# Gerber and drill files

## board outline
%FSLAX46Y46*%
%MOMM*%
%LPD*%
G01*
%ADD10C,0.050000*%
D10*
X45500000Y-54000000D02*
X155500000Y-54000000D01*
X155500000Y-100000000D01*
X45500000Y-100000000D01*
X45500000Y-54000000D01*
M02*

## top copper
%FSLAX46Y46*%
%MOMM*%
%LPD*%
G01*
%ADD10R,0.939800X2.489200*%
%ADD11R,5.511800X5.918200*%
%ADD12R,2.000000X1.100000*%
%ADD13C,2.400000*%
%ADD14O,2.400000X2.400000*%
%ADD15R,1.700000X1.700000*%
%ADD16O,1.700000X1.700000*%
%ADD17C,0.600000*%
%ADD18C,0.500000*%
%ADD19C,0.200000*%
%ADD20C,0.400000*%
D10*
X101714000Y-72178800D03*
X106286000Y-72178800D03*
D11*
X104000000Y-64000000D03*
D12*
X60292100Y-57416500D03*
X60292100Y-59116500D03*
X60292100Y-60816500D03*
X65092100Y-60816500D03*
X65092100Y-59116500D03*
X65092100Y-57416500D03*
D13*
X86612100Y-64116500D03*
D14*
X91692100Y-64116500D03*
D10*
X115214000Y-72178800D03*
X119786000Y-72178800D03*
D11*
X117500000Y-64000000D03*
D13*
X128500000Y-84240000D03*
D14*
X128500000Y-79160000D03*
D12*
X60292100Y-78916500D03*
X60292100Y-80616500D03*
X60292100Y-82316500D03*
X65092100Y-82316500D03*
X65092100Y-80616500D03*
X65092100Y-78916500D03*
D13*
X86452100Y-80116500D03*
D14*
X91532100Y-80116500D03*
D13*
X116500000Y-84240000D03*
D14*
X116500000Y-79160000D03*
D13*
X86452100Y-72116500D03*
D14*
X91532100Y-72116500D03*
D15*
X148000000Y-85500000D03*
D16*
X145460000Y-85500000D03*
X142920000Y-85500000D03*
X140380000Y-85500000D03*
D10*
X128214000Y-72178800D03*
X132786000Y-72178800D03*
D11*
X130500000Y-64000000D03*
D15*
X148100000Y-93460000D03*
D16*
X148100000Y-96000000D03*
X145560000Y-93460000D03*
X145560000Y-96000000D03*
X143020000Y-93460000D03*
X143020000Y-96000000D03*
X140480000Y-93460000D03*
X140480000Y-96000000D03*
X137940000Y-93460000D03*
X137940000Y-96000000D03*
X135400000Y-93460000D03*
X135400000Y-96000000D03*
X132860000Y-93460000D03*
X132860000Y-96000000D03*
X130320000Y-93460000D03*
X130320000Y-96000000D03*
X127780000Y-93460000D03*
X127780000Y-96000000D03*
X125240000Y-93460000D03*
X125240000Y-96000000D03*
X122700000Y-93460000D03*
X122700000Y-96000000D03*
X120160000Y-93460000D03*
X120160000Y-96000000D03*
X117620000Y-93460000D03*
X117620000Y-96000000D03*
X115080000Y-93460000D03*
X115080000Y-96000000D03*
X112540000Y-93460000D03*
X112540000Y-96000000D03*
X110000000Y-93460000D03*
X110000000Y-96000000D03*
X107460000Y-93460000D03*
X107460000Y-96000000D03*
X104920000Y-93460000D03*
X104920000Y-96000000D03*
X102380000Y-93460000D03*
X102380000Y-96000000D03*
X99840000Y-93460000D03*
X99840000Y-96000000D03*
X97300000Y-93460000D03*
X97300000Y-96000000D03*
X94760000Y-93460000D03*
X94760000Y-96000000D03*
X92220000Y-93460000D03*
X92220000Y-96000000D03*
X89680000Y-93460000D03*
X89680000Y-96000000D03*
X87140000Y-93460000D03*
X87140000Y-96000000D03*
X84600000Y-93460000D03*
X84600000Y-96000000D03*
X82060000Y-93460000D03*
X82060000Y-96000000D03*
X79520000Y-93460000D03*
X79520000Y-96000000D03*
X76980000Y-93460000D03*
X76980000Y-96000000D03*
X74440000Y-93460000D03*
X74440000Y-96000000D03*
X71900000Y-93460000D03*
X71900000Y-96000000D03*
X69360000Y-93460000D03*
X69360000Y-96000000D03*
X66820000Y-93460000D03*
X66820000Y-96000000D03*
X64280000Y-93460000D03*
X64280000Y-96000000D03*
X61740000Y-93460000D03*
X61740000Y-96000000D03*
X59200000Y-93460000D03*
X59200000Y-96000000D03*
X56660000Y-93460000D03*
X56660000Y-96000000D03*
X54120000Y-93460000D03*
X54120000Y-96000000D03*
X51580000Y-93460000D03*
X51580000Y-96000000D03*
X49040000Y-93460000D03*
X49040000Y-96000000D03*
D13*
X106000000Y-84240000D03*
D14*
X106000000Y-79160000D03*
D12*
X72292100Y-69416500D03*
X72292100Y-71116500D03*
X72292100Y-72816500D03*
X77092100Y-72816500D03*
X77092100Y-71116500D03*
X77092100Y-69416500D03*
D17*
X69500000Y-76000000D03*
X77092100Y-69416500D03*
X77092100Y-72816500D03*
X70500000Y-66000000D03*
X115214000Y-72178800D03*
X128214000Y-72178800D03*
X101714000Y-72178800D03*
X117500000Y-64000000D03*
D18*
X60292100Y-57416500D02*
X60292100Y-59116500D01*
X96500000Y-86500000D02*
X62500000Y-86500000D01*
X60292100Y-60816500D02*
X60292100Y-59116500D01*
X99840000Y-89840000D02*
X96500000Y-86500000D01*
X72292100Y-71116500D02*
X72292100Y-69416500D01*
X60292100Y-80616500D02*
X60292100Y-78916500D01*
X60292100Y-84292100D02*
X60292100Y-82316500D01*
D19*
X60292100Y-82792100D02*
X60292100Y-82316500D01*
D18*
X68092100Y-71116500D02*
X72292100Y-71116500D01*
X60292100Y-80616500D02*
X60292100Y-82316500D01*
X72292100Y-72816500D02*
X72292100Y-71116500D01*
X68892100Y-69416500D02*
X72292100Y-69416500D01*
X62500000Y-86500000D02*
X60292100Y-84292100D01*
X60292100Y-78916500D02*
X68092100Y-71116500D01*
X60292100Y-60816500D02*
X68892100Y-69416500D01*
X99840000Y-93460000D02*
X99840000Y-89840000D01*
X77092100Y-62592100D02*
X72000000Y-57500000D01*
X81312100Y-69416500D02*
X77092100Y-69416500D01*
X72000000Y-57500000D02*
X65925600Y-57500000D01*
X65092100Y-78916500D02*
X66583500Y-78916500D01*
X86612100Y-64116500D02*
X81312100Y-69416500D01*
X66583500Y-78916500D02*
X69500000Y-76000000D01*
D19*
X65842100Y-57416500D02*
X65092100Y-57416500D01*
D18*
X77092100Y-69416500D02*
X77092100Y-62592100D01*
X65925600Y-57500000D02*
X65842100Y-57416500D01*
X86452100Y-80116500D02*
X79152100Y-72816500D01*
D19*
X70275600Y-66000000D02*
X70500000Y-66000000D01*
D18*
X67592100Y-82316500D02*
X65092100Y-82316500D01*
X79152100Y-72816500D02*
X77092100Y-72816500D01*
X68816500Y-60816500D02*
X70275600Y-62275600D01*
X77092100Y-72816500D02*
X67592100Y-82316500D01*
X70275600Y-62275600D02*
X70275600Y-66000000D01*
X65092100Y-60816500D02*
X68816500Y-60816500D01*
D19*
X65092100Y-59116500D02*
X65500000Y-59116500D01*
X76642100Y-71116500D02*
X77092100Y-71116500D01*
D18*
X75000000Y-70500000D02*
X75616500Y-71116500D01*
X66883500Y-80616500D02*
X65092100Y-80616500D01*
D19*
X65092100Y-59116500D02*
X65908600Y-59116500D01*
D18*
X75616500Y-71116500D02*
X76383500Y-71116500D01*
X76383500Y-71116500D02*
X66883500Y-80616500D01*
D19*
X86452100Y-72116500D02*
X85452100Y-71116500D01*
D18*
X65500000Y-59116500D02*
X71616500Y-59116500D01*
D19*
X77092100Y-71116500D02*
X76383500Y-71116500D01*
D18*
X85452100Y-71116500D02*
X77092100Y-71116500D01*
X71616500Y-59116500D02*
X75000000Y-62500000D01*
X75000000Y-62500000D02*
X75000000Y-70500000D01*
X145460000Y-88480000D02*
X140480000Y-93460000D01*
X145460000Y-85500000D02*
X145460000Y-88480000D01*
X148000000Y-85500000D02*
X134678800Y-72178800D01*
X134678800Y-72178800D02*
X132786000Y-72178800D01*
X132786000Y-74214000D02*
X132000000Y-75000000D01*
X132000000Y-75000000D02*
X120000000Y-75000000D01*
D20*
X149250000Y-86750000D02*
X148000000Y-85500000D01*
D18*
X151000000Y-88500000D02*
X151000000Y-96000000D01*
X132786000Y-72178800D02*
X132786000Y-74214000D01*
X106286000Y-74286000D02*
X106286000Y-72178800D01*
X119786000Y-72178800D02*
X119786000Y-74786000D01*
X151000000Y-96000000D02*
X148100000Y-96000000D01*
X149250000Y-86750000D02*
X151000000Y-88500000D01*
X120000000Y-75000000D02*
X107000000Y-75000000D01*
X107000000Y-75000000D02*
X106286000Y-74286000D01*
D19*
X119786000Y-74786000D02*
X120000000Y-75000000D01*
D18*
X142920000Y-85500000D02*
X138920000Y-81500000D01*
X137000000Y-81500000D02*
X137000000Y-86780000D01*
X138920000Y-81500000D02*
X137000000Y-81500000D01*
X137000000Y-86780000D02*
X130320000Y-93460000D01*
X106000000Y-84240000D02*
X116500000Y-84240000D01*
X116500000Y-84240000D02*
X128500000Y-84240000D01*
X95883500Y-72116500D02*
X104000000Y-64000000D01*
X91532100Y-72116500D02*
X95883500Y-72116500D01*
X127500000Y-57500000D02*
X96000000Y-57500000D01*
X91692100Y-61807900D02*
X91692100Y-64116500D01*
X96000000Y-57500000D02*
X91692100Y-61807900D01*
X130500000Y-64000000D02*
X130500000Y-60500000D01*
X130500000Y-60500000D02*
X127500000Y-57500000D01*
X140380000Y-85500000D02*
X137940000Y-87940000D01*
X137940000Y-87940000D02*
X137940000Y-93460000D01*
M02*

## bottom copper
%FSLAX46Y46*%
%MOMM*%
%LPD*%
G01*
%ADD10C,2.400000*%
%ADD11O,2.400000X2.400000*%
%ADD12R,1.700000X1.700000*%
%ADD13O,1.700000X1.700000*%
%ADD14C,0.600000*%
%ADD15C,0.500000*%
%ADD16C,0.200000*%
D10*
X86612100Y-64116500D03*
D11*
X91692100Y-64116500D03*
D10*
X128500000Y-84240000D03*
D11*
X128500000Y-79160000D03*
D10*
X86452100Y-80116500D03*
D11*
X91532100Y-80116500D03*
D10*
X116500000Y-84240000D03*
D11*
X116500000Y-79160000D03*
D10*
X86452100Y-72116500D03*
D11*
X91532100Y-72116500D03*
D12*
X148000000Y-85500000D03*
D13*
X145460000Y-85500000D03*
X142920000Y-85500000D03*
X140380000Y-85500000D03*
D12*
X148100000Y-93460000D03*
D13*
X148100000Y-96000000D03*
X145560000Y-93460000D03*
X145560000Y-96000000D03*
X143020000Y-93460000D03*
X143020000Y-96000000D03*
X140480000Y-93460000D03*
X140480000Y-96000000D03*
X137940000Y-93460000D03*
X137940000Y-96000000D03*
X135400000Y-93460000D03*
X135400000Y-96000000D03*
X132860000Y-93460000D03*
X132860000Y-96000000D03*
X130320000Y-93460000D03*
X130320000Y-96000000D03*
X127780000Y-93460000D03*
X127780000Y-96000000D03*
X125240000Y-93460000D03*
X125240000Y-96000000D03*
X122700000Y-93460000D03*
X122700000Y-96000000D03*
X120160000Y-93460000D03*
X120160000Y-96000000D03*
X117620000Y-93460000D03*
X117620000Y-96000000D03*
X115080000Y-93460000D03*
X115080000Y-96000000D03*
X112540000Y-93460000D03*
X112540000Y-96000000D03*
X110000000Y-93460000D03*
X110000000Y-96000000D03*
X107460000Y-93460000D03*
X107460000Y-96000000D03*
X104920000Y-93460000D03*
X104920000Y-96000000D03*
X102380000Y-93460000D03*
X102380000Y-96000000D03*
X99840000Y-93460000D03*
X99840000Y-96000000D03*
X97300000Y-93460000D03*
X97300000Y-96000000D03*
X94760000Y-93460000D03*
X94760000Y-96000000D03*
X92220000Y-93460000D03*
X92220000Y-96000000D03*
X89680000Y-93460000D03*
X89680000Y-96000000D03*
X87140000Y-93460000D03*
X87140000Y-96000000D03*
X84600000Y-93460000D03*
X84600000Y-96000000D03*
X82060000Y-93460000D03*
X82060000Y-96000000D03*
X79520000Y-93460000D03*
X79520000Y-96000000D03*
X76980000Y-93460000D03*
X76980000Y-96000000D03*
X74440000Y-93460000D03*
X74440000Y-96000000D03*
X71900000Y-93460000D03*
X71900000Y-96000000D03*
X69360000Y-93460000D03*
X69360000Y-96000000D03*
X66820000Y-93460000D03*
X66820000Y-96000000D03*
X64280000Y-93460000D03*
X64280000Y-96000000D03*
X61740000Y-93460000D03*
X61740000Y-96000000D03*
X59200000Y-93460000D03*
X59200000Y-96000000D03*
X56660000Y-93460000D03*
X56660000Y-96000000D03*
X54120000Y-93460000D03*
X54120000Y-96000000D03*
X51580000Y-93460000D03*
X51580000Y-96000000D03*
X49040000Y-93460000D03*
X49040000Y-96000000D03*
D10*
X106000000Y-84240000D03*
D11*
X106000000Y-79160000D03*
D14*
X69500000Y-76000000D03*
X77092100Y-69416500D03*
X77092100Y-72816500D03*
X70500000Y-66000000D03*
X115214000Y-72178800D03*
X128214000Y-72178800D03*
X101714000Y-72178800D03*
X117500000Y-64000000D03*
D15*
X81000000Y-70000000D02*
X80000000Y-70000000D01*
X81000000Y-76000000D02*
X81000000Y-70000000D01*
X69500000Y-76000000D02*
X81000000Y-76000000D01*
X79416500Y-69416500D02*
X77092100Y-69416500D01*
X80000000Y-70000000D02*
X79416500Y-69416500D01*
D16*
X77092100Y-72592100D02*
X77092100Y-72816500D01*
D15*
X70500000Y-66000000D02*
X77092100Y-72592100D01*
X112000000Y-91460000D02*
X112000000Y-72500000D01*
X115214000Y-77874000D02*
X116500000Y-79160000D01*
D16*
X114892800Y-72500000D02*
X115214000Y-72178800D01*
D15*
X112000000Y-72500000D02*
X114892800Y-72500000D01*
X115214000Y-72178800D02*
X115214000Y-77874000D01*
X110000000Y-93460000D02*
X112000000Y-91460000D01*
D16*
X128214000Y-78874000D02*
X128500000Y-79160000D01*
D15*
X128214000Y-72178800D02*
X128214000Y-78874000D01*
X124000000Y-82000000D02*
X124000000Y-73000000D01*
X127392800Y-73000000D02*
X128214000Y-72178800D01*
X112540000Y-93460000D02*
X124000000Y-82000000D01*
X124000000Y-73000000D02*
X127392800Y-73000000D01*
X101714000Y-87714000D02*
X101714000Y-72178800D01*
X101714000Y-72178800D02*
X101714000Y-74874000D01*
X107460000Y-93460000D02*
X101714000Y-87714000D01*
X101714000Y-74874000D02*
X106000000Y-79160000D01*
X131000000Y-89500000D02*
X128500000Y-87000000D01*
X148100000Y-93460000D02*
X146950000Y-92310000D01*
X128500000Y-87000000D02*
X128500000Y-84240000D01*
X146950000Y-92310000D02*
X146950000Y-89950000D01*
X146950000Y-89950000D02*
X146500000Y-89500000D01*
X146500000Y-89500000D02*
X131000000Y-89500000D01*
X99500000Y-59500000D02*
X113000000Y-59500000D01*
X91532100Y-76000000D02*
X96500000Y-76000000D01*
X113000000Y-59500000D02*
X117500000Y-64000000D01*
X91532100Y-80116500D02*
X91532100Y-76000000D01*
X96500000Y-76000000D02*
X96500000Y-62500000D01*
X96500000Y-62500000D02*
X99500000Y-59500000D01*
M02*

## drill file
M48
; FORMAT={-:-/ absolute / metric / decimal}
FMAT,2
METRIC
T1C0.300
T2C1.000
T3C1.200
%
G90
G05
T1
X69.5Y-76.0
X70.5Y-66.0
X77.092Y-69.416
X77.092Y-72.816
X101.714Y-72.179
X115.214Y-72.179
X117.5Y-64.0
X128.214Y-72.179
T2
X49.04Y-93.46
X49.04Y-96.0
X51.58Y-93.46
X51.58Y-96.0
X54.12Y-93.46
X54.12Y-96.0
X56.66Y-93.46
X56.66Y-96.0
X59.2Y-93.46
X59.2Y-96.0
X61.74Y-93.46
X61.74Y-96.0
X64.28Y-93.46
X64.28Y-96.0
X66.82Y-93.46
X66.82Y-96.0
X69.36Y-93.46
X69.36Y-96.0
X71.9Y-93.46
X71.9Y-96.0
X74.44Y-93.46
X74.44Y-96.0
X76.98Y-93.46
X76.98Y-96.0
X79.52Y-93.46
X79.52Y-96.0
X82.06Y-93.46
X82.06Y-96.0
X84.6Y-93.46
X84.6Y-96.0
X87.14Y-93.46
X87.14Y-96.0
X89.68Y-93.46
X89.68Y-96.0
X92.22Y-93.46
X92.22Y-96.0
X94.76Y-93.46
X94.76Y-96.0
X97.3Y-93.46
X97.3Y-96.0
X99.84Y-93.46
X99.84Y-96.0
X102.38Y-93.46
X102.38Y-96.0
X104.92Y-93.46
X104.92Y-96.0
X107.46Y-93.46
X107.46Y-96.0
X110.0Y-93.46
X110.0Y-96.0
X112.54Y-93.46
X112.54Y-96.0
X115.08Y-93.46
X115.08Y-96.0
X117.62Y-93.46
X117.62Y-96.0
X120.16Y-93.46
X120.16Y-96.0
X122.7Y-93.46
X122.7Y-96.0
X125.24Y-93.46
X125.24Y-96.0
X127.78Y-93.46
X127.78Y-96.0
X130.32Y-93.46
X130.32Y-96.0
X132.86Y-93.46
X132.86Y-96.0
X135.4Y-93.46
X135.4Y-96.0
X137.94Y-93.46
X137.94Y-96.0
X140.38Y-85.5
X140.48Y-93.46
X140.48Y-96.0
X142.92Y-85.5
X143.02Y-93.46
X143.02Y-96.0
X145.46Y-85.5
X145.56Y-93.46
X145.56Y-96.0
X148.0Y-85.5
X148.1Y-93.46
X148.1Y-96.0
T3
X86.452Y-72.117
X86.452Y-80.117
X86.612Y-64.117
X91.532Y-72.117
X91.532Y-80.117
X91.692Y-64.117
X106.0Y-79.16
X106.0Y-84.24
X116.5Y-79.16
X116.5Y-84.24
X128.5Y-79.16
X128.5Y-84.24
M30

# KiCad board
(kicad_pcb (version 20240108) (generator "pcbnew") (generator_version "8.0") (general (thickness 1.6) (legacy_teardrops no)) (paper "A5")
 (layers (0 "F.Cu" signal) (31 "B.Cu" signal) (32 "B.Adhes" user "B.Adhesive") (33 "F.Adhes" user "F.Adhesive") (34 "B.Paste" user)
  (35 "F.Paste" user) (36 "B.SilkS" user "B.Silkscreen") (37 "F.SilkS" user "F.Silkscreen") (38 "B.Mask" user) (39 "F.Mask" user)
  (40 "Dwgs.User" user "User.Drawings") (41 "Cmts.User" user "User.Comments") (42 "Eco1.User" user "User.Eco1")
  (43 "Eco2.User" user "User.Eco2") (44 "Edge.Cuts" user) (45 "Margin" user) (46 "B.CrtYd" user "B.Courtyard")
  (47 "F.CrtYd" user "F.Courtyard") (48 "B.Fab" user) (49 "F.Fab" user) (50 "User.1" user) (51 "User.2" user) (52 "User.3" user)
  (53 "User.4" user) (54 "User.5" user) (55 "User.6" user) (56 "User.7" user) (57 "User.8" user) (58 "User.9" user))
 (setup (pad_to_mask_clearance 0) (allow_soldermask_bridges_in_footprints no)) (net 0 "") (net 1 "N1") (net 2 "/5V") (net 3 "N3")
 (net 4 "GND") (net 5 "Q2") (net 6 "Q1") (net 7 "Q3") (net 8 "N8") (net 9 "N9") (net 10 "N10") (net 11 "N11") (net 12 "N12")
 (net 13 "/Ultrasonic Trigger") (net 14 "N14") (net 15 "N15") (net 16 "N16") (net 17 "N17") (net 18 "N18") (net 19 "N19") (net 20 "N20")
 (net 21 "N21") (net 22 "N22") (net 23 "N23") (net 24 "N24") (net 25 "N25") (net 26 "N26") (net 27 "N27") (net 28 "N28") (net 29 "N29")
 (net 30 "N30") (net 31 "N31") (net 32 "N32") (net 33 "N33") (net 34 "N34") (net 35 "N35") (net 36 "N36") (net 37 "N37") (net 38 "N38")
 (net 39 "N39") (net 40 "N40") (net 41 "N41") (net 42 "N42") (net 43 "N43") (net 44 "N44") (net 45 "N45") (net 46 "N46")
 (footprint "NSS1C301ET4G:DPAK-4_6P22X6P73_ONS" (layer "F.Cu") (at 104 65.7653)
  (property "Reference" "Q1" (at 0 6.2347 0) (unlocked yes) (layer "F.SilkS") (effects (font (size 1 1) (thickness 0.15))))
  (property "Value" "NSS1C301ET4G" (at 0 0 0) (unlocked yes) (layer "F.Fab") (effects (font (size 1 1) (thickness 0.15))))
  (pad "1" smd rect (at -2.286 6.4135) (size 0.9398 2.4892) (layers "F.Cu" "F.Paste" "F.Mask") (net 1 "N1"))
  (pad "2" smd rect (at 2.286 6.4135) (size 0.9398 2.4892) (layers "F.Cu" "F.Paste" "F.Mask") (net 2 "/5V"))
  (pad "3" smd rect (at 0 -1.7653) (size 5.5118 5.9182) (layers "F.Cu" "F.Paste" "F.Mask") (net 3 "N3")))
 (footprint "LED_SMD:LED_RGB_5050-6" (layer "F.Cu") (at 62.6921 59.1165)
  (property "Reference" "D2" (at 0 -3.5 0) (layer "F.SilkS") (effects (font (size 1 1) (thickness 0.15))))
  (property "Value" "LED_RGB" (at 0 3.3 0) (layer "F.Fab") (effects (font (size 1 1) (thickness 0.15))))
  (pad "1" smd rect (at -2.4 -1.7 90) (size 1.1 2) (layers "F.Cu" "F.Paste" "F.Mask") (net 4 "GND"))
  (pad "2" smd rect (at -2.4 0 90) (size 1.1 2) (layers "F.Cu" "F.Paste" "F.Mask") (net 4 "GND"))
  (pad "3" smd rect (at -2.4 1.7 90) (size 1.1 2) (layers "F.Cu" "F.Paste" "F.Mask") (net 4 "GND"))
  (pad "4" smd rect (at 2.4 1.7 90) (size 1.1 2) (layers "F.Cu" "F.Paste" "F.Mask") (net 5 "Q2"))
  (pad "5" smd rect (at 2.4 0 90) (size 1.1 2) (layers "F.Cu" "F.Paste" "F.Mask") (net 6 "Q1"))
  (pad "6" smd rect (at 2.4 -1.7 90) (size 1.1 2) (layers "F.Cu" "F.Paste" "F.Mask") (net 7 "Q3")))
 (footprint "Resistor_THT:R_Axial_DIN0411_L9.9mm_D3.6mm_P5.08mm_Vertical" (layer "F.Cu") (at 86.6121 64.1165)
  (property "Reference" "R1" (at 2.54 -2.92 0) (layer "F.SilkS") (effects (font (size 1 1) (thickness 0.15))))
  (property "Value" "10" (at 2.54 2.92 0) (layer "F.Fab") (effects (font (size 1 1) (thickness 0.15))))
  (pad "1" thru_hole circle (at 0 0) (size 2.4 2.4) (drill 1.2) (layers "*.Cu" "*.Mask") (remove_unused_layers no) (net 7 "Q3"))
  (pad "2" thru_hole oval (at 5.08 0) (size 2.4 2.4) (drill 1.2) (layers "*.Cu" "*.Mask") (remove_unused_layers no) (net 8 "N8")))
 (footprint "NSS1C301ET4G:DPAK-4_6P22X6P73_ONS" (layer "F.Cu") (at 117.5 65.7653)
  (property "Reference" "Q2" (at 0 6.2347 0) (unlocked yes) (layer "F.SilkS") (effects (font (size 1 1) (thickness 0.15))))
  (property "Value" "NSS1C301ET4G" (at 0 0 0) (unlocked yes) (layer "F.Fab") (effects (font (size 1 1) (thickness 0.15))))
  (pad "1" smd rect (at -2.286 6.4135) (size 0.9398 2.4892) (layers "F.Cu" "F.Paste" "F.Mask") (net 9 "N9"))
  (pad "2" smd rect (at 2.286 6.4135) (size 0.9398 2.4892) (layers "F.Cu" "F.Paste" "F.Mask") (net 2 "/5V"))
  (pad "3" smd rect (at 0 -1.7653) (size 5.5118 5.9182) (layers "F.Cu" "F.Paste" "F.Mask") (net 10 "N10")))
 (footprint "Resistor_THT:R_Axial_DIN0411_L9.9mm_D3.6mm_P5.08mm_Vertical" (layer "F.Cu") (at 128.5 84.24 90)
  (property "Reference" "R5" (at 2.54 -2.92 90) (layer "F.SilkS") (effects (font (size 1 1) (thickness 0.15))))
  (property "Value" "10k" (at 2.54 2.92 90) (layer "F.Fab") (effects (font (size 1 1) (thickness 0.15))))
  (pad "1" thru_hole circle (at 0 0 90) (size 2.4 2.4) (drill 1.2) (layers "*.Cu" "*.Mask") (remove_unused_layers no) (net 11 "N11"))
  (pad "2" thru_hole oval (at 5.08 0 90) (size 2.4 2.4) (drill 1.2) (layers "*.Cu" "*.Mask") (remove_unused_layers no) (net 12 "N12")))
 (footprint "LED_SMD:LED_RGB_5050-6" (layer "F.Cu") (at 62.6921 80.6165)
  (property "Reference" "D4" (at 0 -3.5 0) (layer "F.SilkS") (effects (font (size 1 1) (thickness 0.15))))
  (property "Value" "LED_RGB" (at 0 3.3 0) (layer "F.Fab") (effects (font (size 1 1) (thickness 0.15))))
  (pad "1" smd rect (at -2.4 -1.7 90) (size 1.1 2) (layers "F.Cu" "F.Paste" "F.Mask") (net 4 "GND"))
  (pad "2" smd rect (at -2.4 0 90) (size 1.1 2) (layers "F.Cu" "F.Paste" "F.Mask") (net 4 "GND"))
  (pad "3" smd rect (at -2.4 1.7 90) (size 1.1 2) (layers "F.Cu" "F.Paste" "F.Mask") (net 4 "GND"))
  (pad "4" smd rect (at 2.4 1.7 90) (size 1.1 2) (layers "F.Cu" "F.Paste" "F.Mask") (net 5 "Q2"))
  (pad "5" smd rect (at 2.4 0 90) (size 1.1 2) (layers "F.Cu" "F.Paste" "F.Mask") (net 6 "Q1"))
  (pad "6" smd rect (at 2.4 -1.7 90) (size 1.1 2) (layers "F.Cu" "F.Paste" "F.Mask") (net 7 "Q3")))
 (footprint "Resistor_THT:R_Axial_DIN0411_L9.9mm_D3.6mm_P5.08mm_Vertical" (layer "F.Cu") (at 86.4521 80.1165)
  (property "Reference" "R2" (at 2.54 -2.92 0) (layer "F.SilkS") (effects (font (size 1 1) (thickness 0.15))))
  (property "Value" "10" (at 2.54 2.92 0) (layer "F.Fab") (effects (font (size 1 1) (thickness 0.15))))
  (pad "1" thru_hole circle (at 0 0) (size 2.4 2.4) (drill 1.2) (layers "*.Cu" "*.Mask") (remove_unused_layers no) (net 5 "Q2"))
  (pad "2" thru_hole oval (at 5.08 0) (size 2.4 2.4) (drill 1.2) (layers "*.Cu" "*.Mask") (remove_unused_layers no) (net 10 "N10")))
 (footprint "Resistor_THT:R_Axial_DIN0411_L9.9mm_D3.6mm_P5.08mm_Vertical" (layer "F.Cu") (at 116.5 84.24 90)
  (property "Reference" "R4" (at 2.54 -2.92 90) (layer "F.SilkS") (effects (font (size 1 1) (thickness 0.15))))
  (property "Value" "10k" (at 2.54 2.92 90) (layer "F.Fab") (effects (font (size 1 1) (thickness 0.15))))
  (pad "1" thru_hole circle (at 0 0 90) (size 2.4 2.4) (drill 1.2) (layers "*.Cu" "*.Mask") (remove_unused_layers no) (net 11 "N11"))
  (pad "2" thru_hole oval (at 5.08 0 90) (size 2.4 2.4) (drill 1.2) (layers "*.Cu" "*.Mask") (remove_unused_layers no) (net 9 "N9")))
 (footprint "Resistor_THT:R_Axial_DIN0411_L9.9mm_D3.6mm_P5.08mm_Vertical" (layer "F.Cu") (at 86.4521 72.1165)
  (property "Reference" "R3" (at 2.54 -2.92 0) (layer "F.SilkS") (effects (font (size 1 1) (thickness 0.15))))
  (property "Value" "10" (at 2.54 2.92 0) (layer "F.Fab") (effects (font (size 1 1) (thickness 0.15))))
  (pad "1" thru_hole circle (at 0 0) (size 2.4 2.4) (drill 1.2) (layers "*.Cu" "*.Mask") (remove_unused_layers no) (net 6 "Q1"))
  (pad "2" thru_hole oval (at 5.08 0) (size 2.4 2.4) (drill 1.2) (layers "*.Cu" "*.Mask") (remove_unused_layers no) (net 3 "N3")))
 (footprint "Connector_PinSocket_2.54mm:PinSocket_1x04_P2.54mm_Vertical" (layer "F.Cu") (at 148 85.5 -90)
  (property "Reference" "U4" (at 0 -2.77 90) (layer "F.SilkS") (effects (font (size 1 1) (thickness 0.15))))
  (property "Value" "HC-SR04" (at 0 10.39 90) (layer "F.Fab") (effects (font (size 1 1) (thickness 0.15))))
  (pad "1" thru_hole rect (at 0 0 270) (size 1.7 1.7) (drill 1) (layers "*.Cu" "*.Mask") (remove_unused_layers no) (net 2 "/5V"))
  (pad "2" thru_hole oval (at 0 2.54 270) (size 1.7 1.7) (drill 1) (layers "*.Cu" "*.Mask") (remove_unused_layers no)
   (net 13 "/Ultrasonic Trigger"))
  (pad "3" thru_hole oval (at 0 5.08 270) (size 1.7 1.7) (drill 1) (layers "*.Cu" "*.Mask") (remove_unused_layers no) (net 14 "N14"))
  (pad "4" thru_hole oval (at 0 7.62 270) (size 1.7 1.7) (drill 1) (layers "*.Cu" "*.Mask") (remove_unused_layers no) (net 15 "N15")))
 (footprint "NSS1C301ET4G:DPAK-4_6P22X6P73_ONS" (layer "F.Cu") (at 130.5 65.7653)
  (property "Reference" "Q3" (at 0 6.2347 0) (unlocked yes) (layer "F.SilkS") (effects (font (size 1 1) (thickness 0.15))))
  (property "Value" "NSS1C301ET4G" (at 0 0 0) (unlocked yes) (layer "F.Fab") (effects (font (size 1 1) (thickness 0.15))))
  (pad "1" smd rect (at -2.286 6.4135) (size 0.9398 2.4892) (layers "F.Cu" "F.Paste" "F.Mask") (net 12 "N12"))
  (pad "2" smd rect (at 2.286 6.4135) (size 0.9398 2.4892) (layers "F.Cu" "F.Paste" "F.Mask") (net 2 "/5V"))
  (pad "3" smd rect (at 0 -1.7653) (size 5.5118 5.9182) (layers "F.Cu" "F.Paste" "F.Mask") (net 8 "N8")))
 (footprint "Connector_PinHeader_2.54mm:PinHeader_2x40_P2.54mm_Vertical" (layer "F.Cu") (at 148.1 93.46 -90)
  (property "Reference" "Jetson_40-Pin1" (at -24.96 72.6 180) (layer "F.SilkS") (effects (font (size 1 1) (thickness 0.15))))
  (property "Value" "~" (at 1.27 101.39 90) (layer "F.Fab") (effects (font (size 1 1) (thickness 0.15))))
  (pad "1" thru_hole rect (at 0 0 270) (size 1.7 1.7) (drill 1) (layers "*.Cu" "*.Mask") (remove_unused_layers no) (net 11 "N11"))
  (pad "2" thru_hole oval (at 2.54 0 270) (size 1.7 1.7) (drill 1) (layers "*.Cu" "*.Mask") (remove_unused_layers no) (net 2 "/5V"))
  (pad "3" thru_hole oval (at 0 2.54 270) (size 1.7 1.7) (drill 1) (layers "*.Cu" "*.Mask") (remove_unused_layers no) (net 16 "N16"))
  (pad "4" thru_hole oval (at 2.54 2.54 270) (size 1.7 1.7) (drill 1) (layers "*.Cu" "*.Mask") (remove_unused_layers no) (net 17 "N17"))
  (pad "5" thru_hole oval (at 0 5.08 270) (size 1.7 1.7) (drill 1) (layers "*.Cu" "*.Mask") (remove_unused_layers no) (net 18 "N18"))
  (pad "6" thru_hole oval (at 2.54 5.08 270) (size 1.7 1.7) (drill 1) (layers "*.Cu" "*.Mask") (remove_unused_layers no) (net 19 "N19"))
  (pad "7" thru_hole oval (at 0 7.62 270) (size 1.7 1.7) (drill 1) (layers "*.Cu" "*.Mask") (remove_unused_layers no)
   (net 13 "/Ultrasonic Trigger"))
  (pad "8" thru_hole oval (at 2.54 7.62 270) (size 1.7 1.7) (drill 1) (layers "*.Cu" "*.Mask") (remove_unused_layers no) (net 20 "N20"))
  (pad "9" thru_hole oval (at 0 10.16 270) (size 1.7 1.7) (drill 1) (layers "*.Cu" "*.Mask") (remove_unused_layers no) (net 15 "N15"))
  (pad "10" thru_hole oval (at 2.54 10.16 270) (size 1.7 1.7) (drill 1) (layers "*.Cu" "*.Mask") (remove_unused_layers no) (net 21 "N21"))
  (pad "11" thru_hole oval (at 0 12.7 270) (size 1.7 1.7) (drill 1) (layers "*.Cu" "*.Mask") (remove_unused_layers no) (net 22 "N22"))
  (pad "12" thru_hole oval (at 2.54 12.7 270) (size 1.7 1.7) (drill 1) (layers "*.Cu" "*.Mask") (remove_unused_layers no) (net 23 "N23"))
  (pad "13" thru_hole oval (at 0 15.24 270) (size 1.7 1.7) (drill 1) (layers "*.Cu" "*.Mask") (remove_unused_layers no) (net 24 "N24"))
  (pad "14" thru_hole oval (at 2.54 15.24 270) (size 1.7 1.7) (drill 1) (layers "*.Cu" "*.Mask") (remove_unused_layers no) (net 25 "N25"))
  (pad "15" thru_hole oval (at 0 17.78 270) (size 1.7 1.7) (drill 1) (layers "*.Cu" "*.Mask") (remove_unused_layers no) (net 14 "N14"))
  (pad "16" thru_hole oval (at 2.54 17.78 270) (size 1.7 1.7) (drill 1) (layers "*.Cu" "*.Mask") (remove_unused_layers no) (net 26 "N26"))
  (pad "17" thru_hole oval (at 0 20.32 270) (size 1.7 1.7) (drill 1) (layers "*.Cu" "*.Mask") (remove_unused_layers no) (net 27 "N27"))
  (pad "18" thru_hole oval (at 2.54 20.32 270) (size 1.7 1.7) (drill 1) (layers "*.Cu" "*.Mask") (remove_unused_layers no) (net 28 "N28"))
  (pad "19" thru_hole oval (at 0 22.86 270) (size 1.7 1.7) (drill 1) (layers "*.Cu" "*.Mask") (remove_unused_layers no) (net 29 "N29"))
  (pad "20" thru_hole oval (at 2.54 22.86 270) (size 1.7 1.7) (drill 1) (layers "*.Cu" "*.Mask") (remove_unused_layers no) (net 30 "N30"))
  (pad "21" thru_hole oval (at 0 25.4 270) (size 1.7 1.7) (drill 1) (layers "*.Cu" "*.Mask") (remove_unused_layers no) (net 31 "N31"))
  (pad "22" thru_hole oval (at 2.54 25.4 270) (size 1.7 1.7) (drill 1) (layers "*.Cu" "*.Mask") (remove_unused_layers no) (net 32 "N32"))
  (pad "23" thru_hole oval (at 0 27.94 270) (size 1.7 1.7) (drill 1) (layers "*.Cu" "*.Mask") (remove_unused_layers no) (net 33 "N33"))
  (pad "24" thru_hole oval (at 2.54 27.94 270) (size 1.7 1.7) (drill 1) (layers "*.Cu" "*.Mask") (remove_unused_layers no) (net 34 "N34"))
  (pad "25" thru_hole oval (at 0 30.48 270) (size 1.7 1.7) (drill 1) (layers "*.Cu" "*.Mask") (remove_unused_layers no) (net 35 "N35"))
  (pad "26" thru_hole oval (at 2.54 30.48 270) (size 1.7 1.7) (drill 1) (layers "*.Cu" "*.Mask") (remove_unused_layers no) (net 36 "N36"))
  (pad "27" thru_hole oval (at 0 33.02 270) (size 1.7 1.7) (drill 1) (layers "*.Cu" "*.Mask") (remove_unused_layers no) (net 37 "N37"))
  (pad "28" thru_hole oval (at 2.54 33.02 270) (size 1.7 1.7) (drill 1) (layers "*.Cu" "*.Mask") (remove_unused_layers no) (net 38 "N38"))
  (pad "29" thru_hole oval (at 0 35.56 270) (size 1.7 1.7) (drill 1) (layers "*.Cu" "*.Mask") (remove_unused_layers no) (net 12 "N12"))
  (pad "30" thru_hole oval (at 2.54 35.56 270) (size 1.7 1.7) (drill 1) (layers "*.Cu" "*.Mask") (remove_unused_layers no) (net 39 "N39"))
  (pad "31" thru_hole oval (at 0 38.1 270) (size 1.7 1.7) (drill 1) (layers "*.Cu" "*.Mask") (remove_unused_layers no) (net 9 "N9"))
  (pad "32" thru_hole oval (at 2.54 38.1 270) (size 1.7 1.7) (drill 1) (layers "*.Cu" "*.Mask") (remove_unused_layers no) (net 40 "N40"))
  (pad "33" thru_hole oval (at 0 40.64 270) (size 1.7 1.7) (drill 1) (layers "*.Cu" "*.Mask") (remove_unused_layers no) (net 1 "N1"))
  (pad "34" thru_hole oval (at 2.54 40.64 270) (size 1.7 1.7) (drill 1) (layers "*.Cu" "*.Mask") (remove_unused_layers no) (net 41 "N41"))
  (pad "35" thru_hole oval (at 0 43.18 270) (size 1.7 1.7) (drill 1) (layers "*.Cu" "*.Mask") (remove_unused_layers no) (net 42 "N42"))
  (pad "36" thru_hole oval (at 2.54 43.18 270) (size 1.7 1.7) (drill 1) (layers "*.Cu" "*.Mask") (remove_unused_layers no) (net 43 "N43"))
  (pad "37" thru_hole oval (at 0 45.72 270) (size 1.7 1.7) (drill 1) (layers "*.Cu" "*.Mask") (remove_unused_layers no) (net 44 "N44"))
  (pad "38" thru_hole oval (at 2.54 45.72 270) (size 1.7 1.7) (drill 1) (layers "*.Cu" "*.Mask") (remove_unused_layers no) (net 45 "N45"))
  (pad "39" thru_hole oval (at 0 48.26 270) (size 1.7 1.7) (drill 1) (layers "*.Cu" "*.Mask") (remove_unused_layers no) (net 4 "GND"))
  (pad "40" thru_hole oval (at 2.54 48.26 270) (size 1.7 1.7) (drill 1) (layers "*.Cu" "*.Mask") (remove_unused_layers no) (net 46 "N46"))
  (pad "41" thru_hole oval (at 0 50.8 270) (size 1.7 1.7) (drill 1) (layers "*.Cu" "*.Mask") (remove_unused_layers no))
  (pad "42" thru_hole oval (at 2.54 50.8 270) (size 1.7 1.7) (drill 1) (layers "*.Cu" "*.Mask") (remove_unused_layers no))
  (pad "43" thru_hole oval (at 0 53.34 270) (size 1.7 1.7) (drill 1) (layers "*.Cu" "*.Mask") (remove_unused_layers no))
  (pad "44" thru_hole oval (at 2.54 53.34 270) (size 1.7 1.7) (drill 1) (layers "*.Cu" "*.Mask") (remove_unused_layers no))
  (pad "45" thru_hole oval (at 0 55.88 270) (size 1.7 1.7) (drill 1) (layers "*.Cu" "*.Mask") (remove_unused_layers no))
  (pad "46" thru_hole oval (at 2.54 55.88 270) (size 1.7 1.7) (drill 1) (layers "*.Cu" "*.Mask") (remove_unused_layers no))
  (pad "47" thru_hole oval (at 0 58.42 270) (size 1.7 1.7) (drill 1) (layers "*.Cu" "*.Mask") (remove_unused_layers no))
  (pad "48" thru_hole oval (at 2.54 58.42 270) (size 1.7 1.7) (drill 1) (layers "*.Cu" "*.Mask") (remove_unused_layers no))
  (pad "49" thru_hole oval (at 0 60.96 270) (size 1.7 1.7) (drill 1) (layers "*.Cu" "*.Mask") (remove_unused_layers no))
  (pad "50" thru_hole oval (at 2.54 60.96 270) (size 1.7 1.7) (drill 1) (layers "*.Cu" "*.Mask") (remove_unused_layers no))
  (pad "51" thru_hole oval (at 0 63.5 270) (size 1.7 1.7) (drill 1) (layers "*.Cu" "*.Mask") (remove_unused_layers no))
  (pad "52" thru_hole oval (at 2.54 63.5 270) (size 1.7 1.7) (drill 1) (layers "*.Cu" "*.Mask") (remove_unused_layers no))
  (pad "53" thru_hole oval (at 0 66.04 270) (size 1.7 1.7) (drill 1) (layers "*.Cu" "*.Mask") (remove_unused_layers no))
  (pad "54" thru_hole oval (at 2.54 66.04 270) (size 1.7 1.7) (drill 1) (layers "*.Cu" "*.Mask") (remove_unused_layers no))
  (pad "55" thru_hole oval (at 0 68.58 270) (size 1.7 1.7) (drill 1) (layers "*.Cu" "*.Mask") (remove_unused_layers no))
  (pad "56" thru_hole oval (at 2.54 68.58 270) (size 1.7 1.7) (drill 1) (layers "*.Cu" "*.Mask") (remove_unused_layers no))
  (pad "57" thru_hole oval (at 0 71.12 270) (size 1.7 1.7) (drill 1) (layers "*.Cu" "*.Mask") (remove_unused_layers no))
  (pad "58" thru_hole oval (at 2.54 71.12 270) (size 1.7 1.7) (drill 1) (layers "*.Cu" "*.Mask") (remove_unused_layers no))
  (pad "59" thru_hole oval (at 0 73.66 270) (size 1.7 1.7) (drill 1) (layers "*.Cu" "*.Mask") (remove_unused_layers no))
  (pad "60" thru_hole oval (at 2.54 73.66 270) (size 1.7 1.7) (drill 1) (layers "*.Cu" "*.Mask") (remove_unused_layers no))
  (pad "61" thru_hole oval (at 0 76.2 270) (size 1.7 1.7) (drill 1) (layers "*.Cu" "*.Mask") (remove_unused_layers no))
  (pad "62" thru_hole oval (at 2.54 76.2 270) (size 1.7 1.7) (drill 1) (layers "*.Cu" "*.Mask") (remove_unused_layers no))
  (pad "63" thru_hole oval (at 0 78.74 270) (size 1.7 1.7) (drill 1) (layers "*.Cu" "*.Mask") (remove_unused_layers no))
  (pad "64" thru_hole oval (at 2.54 78.74 270) (size 1.7 1.7) (drill 1) (layers "*.Cu" "*.Mask") (remove_unused_layers no))
  (pad "65" thru_hole oval (at 0 81.28 270) (size 1.7 1.7) (drill 1) (layers "*.Cu" "*.Mask") (remove_unused_layers no))
  (pad "66" thru_hole oval (at 2.54 81.28 270) (size 1.7 1.7) (drill 1) (layers "*.Cu" "*.Mask") (remove_unused_layers no))
  (pad "67" thru_hole oval (at 0 83.82 270) (size 1.7 1.7) (drill 1) (layers "*.Cu" "*.Mask") (remove_unused_layers no))
  (pad "68" thru_hole oval (at 2.54 83.82 270) (size 1.7 1.7) (drill 1) (layers "*.Cu" "*.Mask") (remove_unused_layers no))
  (pad "69" thru_hole oval (at 0 86.36 270) (size 1.7 1.7) (drill 1) (layers "*.Cu" "*.Mask") (remove_unused_layers no))
  (pad "70" thru_hole oval (at 2.54 86.36 270) (size 1.7 1.7) (drill 1) (layers "*.Cu" "*.Mask") (remove_unused_layers no))
  (pad "71" thru_hole oval (at 0 88.9 270) (size 1.7 1.7) (drill 1) (layers "*.Cu" "*.Mask") (remove_unused_layers no))
  (pad "72" thru_hole oval (at 2.54 88.9 270) (size 1.7 1.7) (drill 1) (layers "*.Cu" "*.Mask") (remove_unused_layers no))
  (pad "73" thru_hole oval (at 0 91.44 270) (size 1.7 1.7) (drill 1) (layers "*.Cu" "*.Mask") (remove_unused_layers no))
  (pad "74" thru_hole oval (at 2.54 91.44 270) (size 1.7 1.7) (drill 1) (layers "*.Cu" "*.Mask") (remove_unused_layers no))
  (pad "75" thru_hole oval (at 0 93.98 270) (size 1.7 1.7) (drill 1) (layers "*.Cu" "*.Mask") (remove_unused_layers no))
  (pad "76" thru_hole oval (at 2.54 93.98 270) (size 1.7 1.7) (drill 1) (layers "*.Cu" "*.Mask") (remove_unused_layers no))
  (pad "77" thru_hole oval (at 0 96.52 270) (size 1.7 1.7) (drill 1) (layers "*.Cu" "*.Mask") (remove_unused_layers no))
  (pad "78" thru_hole oval (at 2.54 96.52 270) (size 1.7 1.7) (drill 1) (layers "*.Cu" "*.Mask") (remove_unused_layers no))
  (pad "79" thru_hole oval (at 0 99.06 270) (size 1.7 1.7) (drill 1) (layers "*.Cu" "*.Mask") (remove_unused_layers no))
  (pad "80" thru_hole oval (at 2.54 99.06 270) (size 1.7 1.7) (drill 1) (layers "*.Cu" "*.Mask") (remove_unused_layers no)))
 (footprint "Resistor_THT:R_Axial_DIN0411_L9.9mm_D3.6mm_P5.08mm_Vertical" (layer "F.Cu") (at 106 84.24 90)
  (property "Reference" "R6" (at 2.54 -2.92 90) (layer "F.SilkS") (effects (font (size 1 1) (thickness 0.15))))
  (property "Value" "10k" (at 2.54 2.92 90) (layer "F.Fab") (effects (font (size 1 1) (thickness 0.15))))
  (pad "1" thru_hole circle (at 0 0 90) (size 2.4 2.4) (drill 1.2) (layers "*.Cu" "*.Mask") (remove_unused_layers no) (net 11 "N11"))
  (pad "2" thru_hole oval (at 5.08 0 90) (size 2.4 2.4) (drill 1.2) (layers "*.Cu" "*.Mask") (remove_unused_layers no) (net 1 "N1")))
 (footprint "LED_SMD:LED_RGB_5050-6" (layer "F.Cu") (at 74.6921 71.1165)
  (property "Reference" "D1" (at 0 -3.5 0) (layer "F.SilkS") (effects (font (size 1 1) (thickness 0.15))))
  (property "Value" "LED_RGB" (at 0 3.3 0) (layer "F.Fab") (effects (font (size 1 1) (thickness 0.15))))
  (pad "1" smd rect (at -2.4 -1.7 90) (size 1.1 2) (layers "F.Cu" "F.Paste" "F.Mask") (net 4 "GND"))
  (pad "2" smd rect (at -2.4 0 90) (size 1.1 2) (layers "F.Cu" "F.Paste" "F.Mask") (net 4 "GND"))
  (pad "3" smd rect (at -2.4 1.7 90) (size 1.1 2) (layers "F.Cu" "F.Paste" "F.Mask") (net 4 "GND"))
  (pad "4" smd rect (at 2.4 1.7 90) (size 1.1 2) (layers "F.Cu" "F.Paste" "F.Mask") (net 5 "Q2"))
  (pad "5" smd rect (at 2.4 0 90) (size 1.1 2) (layers "F.Cu" "F.Paste" "F.Mask") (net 6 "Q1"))
  (pad "6" smd rect (at 2.4 -1.7 90) (size 1.1 2) (layers "F.Cu" "F.Paste" "F.Mask") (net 7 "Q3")))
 (gr_rect (start 45.5 54) (end 155.5 100) (stroke (width 0.05) (type default)) (fill none) (layer "Edge.Cuts"))
 (segment (start 60.2921 57.4165) (end 60.2921 59.1165) (width 0.5) (layer "F.Cu") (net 4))
 (segment (start 96.5 86.5) (end 62.5 86.5) (width 0.5) (layer "F.Cu") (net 4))
 (segment (start 60.2921 60.8165) (end 60.2921 59.1165) (width 0.5) (layer "F.Cu") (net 4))
 (segment (start 99.84 89.84) (end 96.5 86.5) (width 0.5) (layer "F.Cu") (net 4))
 (segment (start 72.2921 71.1165) (end 72.2921 69.4165) (width 0.5) (layer "F.Cu") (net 4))
 (segment (start 60.2921 80.6165) (end 60.2921 78.9165) (width 0.5) (layer "F.Cu") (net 4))
 (segment (start 60.2921 84.2921) (end 60.2921 82.3165) (width 0.5) (layer "F.Cu") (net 4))
 (segment (start 60.2921 82.7921) (end 60.2921 82.3165) (width 0.2) (layer "F.Cu") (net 4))
 (segment (start 68.0921 71.1165) (end 72.2921 71.1165) (width 0.5) (layer "F.Cu") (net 4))
 (segment (start 60.2921 80.6165) (end 60.2921 82.3165) (width 0.5) (layer "F.Cu") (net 4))
 (segment (start 72.2921 72.8165) (end 72.2921 71.1165) (width 0.5) (layer "F.Cu") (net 4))
 (segment (start 68.8921 69.4165) (end 72.2921 69.4165) (width 0.5) (layer "F.Cu") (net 4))
 (segment (start 62.5 86.5) (end 60.2921 84.2921) (width 0.5) (layer "F.Cu") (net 4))
 (segment (start 60.2921 78.9165) (end 68.0921 71.1165) (width 0.5) (layer "F.Cu") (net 4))
 (segment (start 60.2921 60.8165) (end 68.8921 69.4165) (width 0.5) (layer "F.Cu") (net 4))
 (segment (start 99.84 93.46) (end 99.84 89.84) (width 0.5) (layer "F.Cu") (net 4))
 (segment (start 77.0921 62.5921) (end 72 57.5) (width 0.5) (layer "F.Cu") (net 7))
 (segment (start 81.3121 69.4165) (end 77.0921 69.4165) (width 0.5) (layer "F.Cu") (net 7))
 (segment (start 72 57.5) (end 65.9256 57.5) (width 0.5) (layer "F.Cu") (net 7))
 (segment (start 65.0921 78.9165) (end 66.5835 78.9165) (width 0.5) (layer "F.Cu") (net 7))
 (segment (start 86.6121 64.1165) (end 81.3121 69.4165) (width 0.5) (layer "F.Cu") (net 7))
 (segment (start 66.5835 78.9165) (end 69.5 76) (width 0.5) (layer "F.Cu") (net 7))
 (segment (start 65.8421 57.4165) (end 65.0921 57.4165) (width 0.2) (layer "F.Cu") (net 7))
 (segment (start 77.0921 69.4165) (end 77.0921 62.5921) (width 0.5) (layer "F.Cu") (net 7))
 (segment (start 65.9256 57.5) (end 65.8421 57.4165) (width 0.5) (layer "F.Cu") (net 7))
 (via (at 69.5 76) (size 0.6) (drill 0.3) (layers "F.Cu" "B.Cu") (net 7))
 (via (at 77.0921 69.4165) (size 0.6) (drill 0.3) (layers "F.Cu" "B.Cu") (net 7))
 (segment (start 81 70) (end 80 70) (width 0.5) (layer "B.Cu") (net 7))
 (segment (start 81 76) (end 81 70) (width 0.5) (layer "B.Cu") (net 7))
 (segment (start 69.5 76) (end 81 76) (width 0.5) (layer "B.Cu") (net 7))
 (segment (start 79.4165 69.4165) (end 77.0921 69.4165) (width 0.5) (layer "B.Cu") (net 7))
 (segment (start 80 70) (end 79.4165 69.4165) (width 0.5) (layer "B.Cu") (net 7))
 (segment (start 86.4521 80.1165) (end 79.1521 72.8165) (width 0.5) (layer "F.Cu") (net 5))
 (segment (start 70.2756 66) (end 70.5 66) (width 0.2) (layer "F.Cu") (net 5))
 (segment (start 67.5921 82.3165) (end 65.0921 82.3165) (width 0.5) (layer "F.Cu") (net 5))
 (segment (start 79.1521 72.8165) (end 77.0921 72.8165) (width 0.5) (layer "F.Cu") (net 5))
 (segment (start 68.8165 60.8165) (end 70.2756 62.2756) (width 0.5) (layer "F.Cu") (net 5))
 (segment (start 77.0921 72.8165) (end 67.5921 82.3165) (width 0.5) (layer "F.Cu") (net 5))
 (segment (start 70.2756 62.2756) (end 70.2756 66) (width 0.5) (layer "F.Cu") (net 5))
 (segment (start 65.0921 60.8165) (end 68.8165 60.8165) (width 0.5) (layer "F.Cu") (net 5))
 (via (at 77.0921 72.8165) (size 0.6) (drill 0.3) (layers "F.Cu" "B.Cu") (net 5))
 (via (at 70.5 66) (size 0.6) (drill 0.3) (layers "F.Cu" "B.Cu") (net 5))
 (segment (start 77.0921 72.5921) (end 77.0921 72.8165) (width 0.2) (layer "B.Cu") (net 5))
 (segment (start 70.5 66) (end 77.0921 72.5921) (width 0.5) (layer "B.Cu") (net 5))
 (segment (start 65.0921 59.1165) (end 65.5 59.1165) (width 0.2) (layer "F.Cu") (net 6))
 (segment (start 76.6421 71.1165) (end 77.0921 71.1165) (width 0.2) (layer "F.Cu") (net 6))
 (segment (start 75 70.5) (end 75.6165 71.1165) (width 0.5) (layer "F.Cu") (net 6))
 (segment (start 66.8835 80.6165) (end 65.0921 80.6165) (width 0.5) (layer "F.Cu") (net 6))
 (segment (start 65.0921 59.1165) (end 65.9086 59.1165) (width 0.2) (layer "F.Cu") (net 6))
 (segment (start 75.6165 71.1165) (end 76.3835 71.1165) (width 0.5) (layer "F.Cu") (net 6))
 (segment (start 76.3835 71.1165) (end 66.8835 80.6165) (width 0.5) (layer "F.Cu") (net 6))
 (segment (start 86.4521 72.1165) (end 85.4521 71.1165) (width 0.2) (layer "F.Cu") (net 6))
 (segment (start 65.5 59.1165) (end 71.6165 59.1165) (width 0.5) (layer "F.Cu") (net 6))
 (segment (start 77.0921 71.1165) (end 76.3835 71.1165) (width 0.2) (layer "F.Cu") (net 6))
 (segment (start 85.4521 71.1165) (end 77.0921 71.1165) (width 0.5) (layer "F.Cu") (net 6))
 (segment (start 71.6165 59.1165) (end 75 62.5) (width 0.5) (layer "F.Cu") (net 6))
 (segment (start 75 62.5) (end 75 70.5) (width 0.5) (layer "F.Cu") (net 6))
 (via (at 115.214 72.1788) (size 0.6) (drill 0.3) (layers "F.Cu" "B.Cu") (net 9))
 (segment (start 112 91.46) (end 112 72.5) (width 0.5) (layer "B.Cu") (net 9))
 (segment (start 115.214 77.874) (end 116.5 79.16) (width 0.5) (layer "B.Cu") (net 9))
 (segment (start 114.8928 72.5) (end 115.214 72.1788) (width 0.2) (layer "B.Cu") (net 9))
 (segment (start 112 72.5) (end 114.8928 72.5) (width 0.5) (layer "B.Cu") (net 9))
 (segment (start 115.214 72.1788) (end 115.214 77.874) (width 0.5) (layer "B.Cu") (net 9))
 (segment (start 110 93.46) (end 112 91.46) (width 0.5) (layer "B.Cu") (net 9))
 (via (at 128.214 72.1788) (size 0.6) (drill 0.3) (layers "F.Cu" "B.Cu") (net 12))
 (segment (start 128.214 78.874) (end 128.5 79.16) (width 0.2) (layer "B.Cu") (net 12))
 (segment (start 128.214 72.1788) (end 128.214 78.874) (width 0.5) (layer "B.Cu") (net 12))
 (segment (start 124 82) (end 124 73) (width 0.5) (layer "B.Cu") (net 12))
 (segment (start 127.3928 73) (end 128.214 72.1788) (width 0.5) (layer "B.Cu") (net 12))
 (segment (start 112.54 93.46) (end 124 82) (width 0.5) (layer "B.Cu") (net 12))
 (segment (start 124 73) (end 127.3928 73) (width 0.5) (layer "B.Cu") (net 12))
 (segment (start 145.46 88.48) (end 140.48 93.46) (width 0.5) (layer "F.Cu") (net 13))
 (segment (start 145.46 85.5) (end 145.46 88.48) (width 0.5) (layer "F.Cu") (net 13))
 (segment (start 148 85.5) (end 134.6788 72.1788) (width 0.5) (layer "F.Cu") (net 2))
 (segment (start 134.6788 72.1788) (end 132.786 72.1788) (width 0.5) (layer "F.Cu") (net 2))
 (segment (start 132.786 74.214) (end 132 75) (width 0.5) (layer "F.Cu") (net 2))
 (segment (start 132 75) (end 120 75) (width 0.5) (layer "F.Cu") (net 2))
 (segment (start 149.25 86.75) (end 148 85.5) (width 0.4) (layer "F.Cu") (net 2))
 (segment (start 151 88.5) (end 151 96) (width 0.5) (layer "F.Cu") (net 2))
 (segment (start 132.786 72.1788) (end 132.786 74.214) (width 0.5) (layer "F.Cu") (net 2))
 (segment (start 106.286 74.286) (end 106.286 72.1788) (width 0.5) (layer "F.Cu") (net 2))
 (segment (start 119.786 72.1788) (end 119.786 74.786) (width 0.5) (layer "F.Cu") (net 2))
 (segment (start 151 96) (end 148.1 96) (width 0.5) (layer "F.Cu") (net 2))
 (segment (start 149.25 86.75) (end 151 88.5) (width 0.5) (layer "F.Cu") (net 2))
 (segment (start 120 75) (end 107 75) (width 0.5) (layer "F.Cu") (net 2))
 (segment (start 107 75) (end 106.286 74.286) (width 0.5) (layer "F.Cu") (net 2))
 (segment (start 119.786 74.786) (end 120 75) (width 0.2) (layer "F.Cu") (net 2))
 (via (at 101.714 72.1788) (size 0.6) (drill 0.3) (layers "F.Cu" "B.Cu") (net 1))
 (segment (start 101.714 87.714) (end 101.714 72.1788) (width 0.5) (layer "B.Cu") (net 1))
 (segment (start 101.714 72.1788) (end 101.714 74.874) (width 0.5) (layer "B.Cu") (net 1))
 (segment (start 107.46 93.46) (end 101.714 87.714) (width 0.5) (layer "B.Cu") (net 1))
 (segment (start 101.714 74.874) (end 106 79.16) (width 0.5) (layer "B.Cu") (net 1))
 (segment (start 142.92 85.5) (end 138.92 81.5) (width 0.5) (layer "F.Cu") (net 14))
 (segment (start 137 81.5) (end 137 86.78) (width 0.5) (layer "F.Cu") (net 14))
 (segment (start 138.92 81.5) (end 137 81.5) (width 0.5) (layer "F.Cu") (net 14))
 (segment (start 137 86.78) (end 130.32 93.46) (width 0.5) (layer "F.Cu") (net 14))
 (segment (start 106 84.24) (end 116.5 84.24) (width 0.5) (layer "F.Cu") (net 11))
 (segment (start 116.5 84.24) (end 128.5 84.24) (width 0.5) (layer "F.Cu") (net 11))
 (segment (start 131 89.5) (end 128.5 87) (width 0.5) (layer "B.Cu") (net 11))
 (segment (start 148.1 93.46) (end 146.95 92.31) (width 0.5) (layer "B.Cu") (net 11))
 (segment (start 128.5 87) (end 128.5 84.24) (width 0.5) (layer "B.Cu") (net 11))
 (segment (start 146.95 92.31) (end 146.95 89.95) (width 0.5) (layer "B.Cu") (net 11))
 (segment (start 146.95 89.95) (end 146.5 89.5) (width 0.5) (layer "B.Cu") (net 11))
 (segment (start 146.5 89.5) (end 131 89.5) (width 0.5) (layer "B.Cu") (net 11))
 (segment (start 95.8835 72.1165) (end 104 64) (width 0.5) (layer "F.Cu") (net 3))
 (segment (start 91.5321 72.1165) (end 95.8835 72.1165) (width 0.5) (layer "F.Cu") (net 3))
 (via (at 117.5 64) (size 0.6) (drill 0.3) (layers "F.Cu" "B.Cu") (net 10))
 (segment (start 99.5 59.5) (end 113 59.5) (width 0.5) (layer "B.Cu") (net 10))
 (segment (start 91.5321 76) (end 96.5 76) (width 0.5) (layer "B.Cu") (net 10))
 (segment (start 113 59.5) (end 117.5 64) (width 0.5) (layer "B.Cu") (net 10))
 (segment (start 91.5321 80.1165) (end 91.5321 76) (width 0.5) (layer "B.Cu") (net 10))
 (segment (start 96.5 76) (end 96.5 62.5) (width 0.5) (layer "B.Cu") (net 10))
 (segment (start 96.5 62.5) (end 99.5 59.5) (width 0.5) (layer "B.Cu") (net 10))
 (segment (start 127.5 57.5) (end 96 57.5) (width 0.5) (layer "F.Cu") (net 8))
 (segment (start 91.6921 61.8079) (end 91.6921 64.1165) (width 0.5) (layer "F.Cu") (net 8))
 (segment (start 96 57.5) (end 91.6921 61.8079) (width 0.5) (layer "F.Cu") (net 8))
 (segment (start 130.5 64) (end 130.5 60.5) (width 0.5) (layer "F.Cu") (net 8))
 (segment (start 130.5 60.5) (end 127.5 57.5) (width 0.5) (layer "F.Cu") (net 8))
 (segment (start 140.38 85.5) (end 137.94 87.94) (width 0.5) (layer "F.Cu") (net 15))
 (segment (start 137.94 87.94) (end 137.94 93.46) (width 0.5) (layer "F.Cu") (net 15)))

